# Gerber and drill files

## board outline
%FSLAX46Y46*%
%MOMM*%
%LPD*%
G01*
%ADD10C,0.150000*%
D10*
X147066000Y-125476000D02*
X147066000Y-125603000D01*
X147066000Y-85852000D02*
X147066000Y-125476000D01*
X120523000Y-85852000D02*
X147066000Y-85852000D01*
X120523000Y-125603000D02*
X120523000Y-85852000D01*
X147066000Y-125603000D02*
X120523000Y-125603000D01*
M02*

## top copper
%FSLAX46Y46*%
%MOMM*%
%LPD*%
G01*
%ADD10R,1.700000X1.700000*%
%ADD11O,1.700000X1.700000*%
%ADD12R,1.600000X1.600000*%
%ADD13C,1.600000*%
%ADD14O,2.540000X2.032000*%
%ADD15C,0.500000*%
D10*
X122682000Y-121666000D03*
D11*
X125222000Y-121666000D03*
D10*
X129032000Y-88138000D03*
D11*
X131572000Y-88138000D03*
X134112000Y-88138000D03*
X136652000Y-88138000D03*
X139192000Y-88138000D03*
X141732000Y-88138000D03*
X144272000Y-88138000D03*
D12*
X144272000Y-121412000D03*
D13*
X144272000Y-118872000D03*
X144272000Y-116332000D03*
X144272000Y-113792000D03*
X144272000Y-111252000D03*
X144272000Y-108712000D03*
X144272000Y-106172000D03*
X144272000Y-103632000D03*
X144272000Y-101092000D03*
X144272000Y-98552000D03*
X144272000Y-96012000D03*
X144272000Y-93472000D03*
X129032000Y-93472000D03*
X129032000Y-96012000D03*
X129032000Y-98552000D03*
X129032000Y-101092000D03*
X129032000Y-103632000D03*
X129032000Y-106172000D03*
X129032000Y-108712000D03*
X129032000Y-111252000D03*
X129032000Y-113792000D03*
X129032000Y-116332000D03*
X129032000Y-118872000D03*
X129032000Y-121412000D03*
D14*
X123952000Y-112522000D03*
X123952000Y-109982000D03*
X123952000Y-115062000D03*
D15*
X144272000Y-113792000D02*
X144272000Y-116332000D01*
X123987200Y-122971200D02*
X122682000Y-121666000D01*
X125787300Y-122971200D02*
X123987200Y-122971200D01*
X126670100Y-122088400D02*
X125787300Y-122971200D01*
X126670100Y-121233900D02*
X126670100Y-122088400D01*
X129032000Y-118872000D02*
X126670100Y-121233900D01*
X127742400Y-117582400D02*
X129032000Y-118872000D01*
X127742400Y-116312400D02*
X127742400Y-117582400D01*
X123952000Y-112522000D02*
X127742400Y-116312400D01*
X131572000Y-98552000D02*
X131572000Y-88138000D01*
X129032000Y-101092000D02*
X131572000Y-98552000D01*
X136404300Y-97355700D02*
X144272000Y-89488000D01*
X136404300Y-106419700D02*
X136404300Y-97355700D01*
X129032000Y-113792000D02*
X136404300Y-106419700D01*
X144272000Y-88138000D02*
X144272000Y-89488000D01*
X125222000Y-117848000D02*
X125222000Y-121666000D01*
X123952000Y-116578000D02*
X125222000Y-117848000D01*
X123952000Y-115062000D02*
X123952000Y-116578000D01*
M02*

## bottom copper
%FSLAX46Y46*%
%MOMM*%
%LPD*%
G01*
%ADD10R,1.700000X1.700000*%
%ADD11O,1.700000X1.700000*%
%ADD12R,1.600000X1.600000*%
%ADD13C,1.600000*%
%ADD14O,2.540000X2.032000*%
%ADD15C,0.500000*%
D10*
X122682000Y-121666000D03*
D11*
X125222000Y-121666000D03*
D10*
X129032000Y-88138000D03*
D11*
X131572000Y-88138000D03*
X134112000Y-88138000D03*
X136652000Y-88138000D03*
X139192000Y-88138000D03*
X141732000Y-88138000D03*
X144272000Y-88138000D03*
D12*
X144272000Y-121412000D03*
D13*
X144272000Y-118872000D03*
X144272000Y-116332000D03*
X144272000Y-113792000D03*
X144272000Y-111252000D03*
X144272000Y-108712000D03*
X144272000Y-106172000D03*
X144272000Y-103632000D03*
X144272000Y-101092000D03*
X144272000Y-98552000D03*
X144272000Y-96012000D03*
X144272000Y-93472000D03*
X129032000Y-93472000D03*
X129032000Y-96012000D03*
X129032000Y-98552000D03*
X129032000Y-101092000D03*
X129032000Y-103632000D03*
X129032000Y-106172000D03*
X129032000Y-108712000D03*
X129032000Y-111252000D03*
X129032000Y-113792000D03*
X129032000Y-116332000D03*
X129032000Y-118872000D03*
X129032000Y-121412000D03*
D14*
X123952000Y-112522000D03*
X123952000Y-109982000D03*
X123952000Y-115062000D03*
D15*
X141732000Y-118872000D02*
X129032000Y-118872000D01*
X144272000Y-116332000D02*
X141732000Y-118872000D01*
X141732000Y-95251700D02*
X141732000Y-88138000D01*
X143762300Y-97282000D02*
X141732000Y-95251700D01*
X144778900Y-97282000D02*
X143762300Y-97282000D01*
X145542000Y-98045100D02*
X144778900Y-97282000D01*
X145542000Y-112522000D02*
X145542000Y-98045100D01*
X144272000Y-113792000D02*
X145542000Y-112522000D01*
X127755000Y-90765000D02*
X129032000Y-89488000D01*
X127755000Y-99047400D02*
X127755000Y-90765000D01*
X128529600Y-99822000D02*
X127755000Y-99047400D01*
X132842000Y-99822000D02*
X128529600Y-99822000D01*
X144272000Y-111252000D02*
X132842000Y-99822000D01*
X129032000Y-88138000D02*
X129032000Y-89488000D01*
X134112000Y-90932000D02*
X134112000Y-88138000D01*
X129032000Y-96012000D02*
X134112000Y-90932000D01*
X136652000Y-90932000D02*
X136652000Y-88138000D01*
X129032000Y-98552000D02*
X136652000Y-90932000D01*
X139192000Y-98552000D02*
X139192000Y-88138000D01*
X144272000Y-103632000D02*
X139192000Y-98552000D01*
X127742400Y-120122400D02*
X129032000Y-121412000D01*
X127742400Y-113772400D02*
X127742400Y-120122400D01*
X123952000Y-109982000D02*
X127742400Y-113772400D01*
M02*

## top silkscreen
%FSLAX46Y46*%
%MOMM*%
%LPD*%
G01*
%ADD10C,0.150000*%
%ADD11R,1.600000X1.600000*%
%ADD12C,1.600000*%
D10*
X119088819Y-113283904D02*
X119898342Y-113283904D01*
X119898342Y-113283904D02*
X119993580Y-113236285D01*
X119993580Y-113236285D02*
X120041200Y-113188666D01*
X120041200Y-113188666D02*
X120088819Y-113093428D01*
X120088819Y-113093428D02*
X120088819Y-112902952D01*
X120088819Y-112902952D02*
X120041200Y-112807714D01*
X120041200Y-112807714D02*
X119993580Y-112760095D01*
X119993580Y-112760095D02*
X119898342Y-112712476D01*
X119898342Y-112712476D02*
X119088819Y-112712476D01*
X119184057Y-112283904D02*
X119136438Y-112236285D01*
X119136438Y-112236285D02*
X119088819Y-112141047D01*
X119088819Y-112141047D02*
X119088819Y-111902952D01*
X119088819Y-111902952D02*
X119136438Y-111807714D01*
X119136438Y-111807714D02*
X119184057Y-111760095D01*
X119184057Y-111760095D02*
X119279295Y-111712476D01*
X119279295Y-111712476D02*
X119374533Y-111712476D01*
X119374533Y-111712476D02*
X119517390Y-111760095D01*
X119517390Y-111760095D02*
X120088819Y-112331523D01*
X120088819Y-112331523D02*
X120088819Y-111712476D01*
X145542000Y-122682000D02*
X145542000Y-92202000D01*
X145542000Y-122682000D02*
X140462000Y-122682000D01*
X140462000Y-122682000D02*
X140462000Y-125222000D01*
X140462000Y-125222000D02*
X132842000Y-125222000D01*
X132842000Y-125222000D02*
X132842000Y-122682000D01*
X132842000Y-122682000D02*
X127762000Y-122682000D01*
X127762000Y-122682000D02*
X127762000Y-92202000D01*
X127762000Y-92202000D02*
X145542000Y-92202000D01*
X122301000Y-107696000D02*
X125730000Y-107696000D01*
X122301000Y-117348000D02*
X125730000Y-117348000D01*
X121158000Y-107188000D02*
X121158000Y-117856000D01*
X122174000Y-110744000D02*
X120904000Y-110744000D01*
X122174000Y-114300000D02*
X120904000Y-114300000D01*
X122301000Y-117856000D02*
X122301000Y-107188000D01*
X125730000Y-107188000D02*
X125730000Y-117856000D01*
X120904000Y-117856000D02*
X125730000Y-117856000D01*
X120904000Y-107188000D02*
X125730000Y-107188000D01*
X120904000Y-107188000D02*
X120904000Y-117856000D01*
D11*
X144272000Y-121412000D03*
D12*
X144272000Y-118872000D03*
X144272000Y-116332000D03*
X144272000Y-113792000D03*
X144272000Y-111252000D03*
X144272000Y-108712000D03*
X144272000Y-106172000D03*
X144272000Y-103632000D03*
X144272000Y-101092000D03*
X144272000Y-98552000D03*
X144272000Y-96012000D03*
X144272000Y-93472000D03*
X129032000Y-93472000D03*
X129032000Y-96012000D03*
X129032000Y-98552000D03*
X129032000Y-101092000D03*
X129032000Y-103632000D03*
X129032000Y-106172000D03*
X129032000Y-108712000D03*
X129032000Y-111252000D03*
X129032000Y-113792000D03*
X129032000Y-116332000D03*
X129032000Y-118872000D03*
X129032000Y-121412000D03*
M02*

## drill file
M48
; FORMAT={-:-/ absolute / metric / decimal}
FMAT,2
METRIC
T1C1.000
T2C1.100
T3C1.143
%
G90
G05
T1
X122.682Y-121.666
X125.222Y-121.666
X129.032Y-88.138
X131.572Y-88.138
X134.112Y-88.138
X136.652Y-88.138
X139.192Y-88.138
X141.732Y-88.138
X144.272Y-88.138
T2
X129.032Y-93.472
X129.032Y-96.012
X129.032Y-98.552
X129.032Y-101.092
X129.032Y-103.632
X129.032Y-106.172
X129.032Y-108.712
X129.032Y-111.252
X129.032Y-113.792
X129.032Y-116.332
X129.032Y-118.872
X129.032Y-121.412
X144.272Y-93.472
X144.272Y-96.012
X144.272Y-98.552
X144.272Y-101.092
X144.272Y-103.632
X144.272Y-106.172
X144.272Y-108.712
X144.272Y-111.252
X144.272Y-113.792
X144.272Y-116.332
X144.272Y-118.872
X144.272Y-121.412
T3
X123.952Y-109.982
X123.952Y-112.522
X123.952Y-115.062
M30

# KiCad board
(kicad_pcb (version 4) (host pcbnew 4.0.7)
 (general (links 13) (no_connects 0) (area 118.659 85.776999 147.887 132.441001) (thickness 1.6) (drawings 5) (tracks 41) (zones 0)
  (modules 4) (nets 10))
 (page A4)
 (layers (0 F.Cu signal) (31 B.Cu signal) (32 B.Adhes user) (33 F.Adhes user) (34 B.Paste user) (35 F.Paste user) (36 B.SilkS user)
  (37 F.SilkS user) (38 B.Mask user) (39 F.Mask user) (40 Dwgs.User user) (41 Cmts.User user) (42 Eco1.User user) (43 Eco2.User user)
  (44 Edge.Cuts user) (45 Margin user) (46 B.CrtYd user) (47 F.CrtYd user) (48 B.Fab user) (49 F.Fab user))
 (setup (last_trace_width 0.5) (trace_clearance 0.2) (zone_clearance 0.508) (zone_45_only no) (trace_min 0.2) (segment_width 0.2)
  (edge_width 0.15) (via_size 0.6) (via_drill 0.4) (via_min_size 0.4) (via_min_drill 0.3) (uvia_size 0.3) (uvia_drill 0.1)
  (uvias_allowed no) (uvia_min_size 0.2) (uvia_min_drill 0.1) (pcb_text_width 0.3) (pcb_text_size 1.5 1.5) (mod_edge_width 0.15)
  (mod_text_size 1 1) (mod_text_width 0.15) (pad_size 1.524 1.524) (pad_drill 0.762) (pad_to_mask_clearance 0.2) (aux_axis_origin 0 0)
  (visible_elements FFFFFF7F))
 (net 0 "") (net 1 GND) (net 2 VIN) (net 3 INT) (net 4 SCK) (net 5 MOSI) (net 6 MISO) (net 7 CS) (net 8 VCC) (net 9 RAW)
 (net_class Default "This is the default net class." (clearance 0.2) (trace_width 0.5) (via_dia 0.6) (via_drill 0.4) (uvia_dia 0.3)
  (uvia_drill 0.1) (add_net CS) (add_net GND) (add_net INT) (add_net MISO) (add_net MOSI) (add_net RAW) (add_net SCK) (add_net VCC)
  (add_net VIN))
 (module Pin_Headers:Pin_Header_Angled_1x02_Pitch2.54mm (layer B.Cu) (at 122.682 121.666 270)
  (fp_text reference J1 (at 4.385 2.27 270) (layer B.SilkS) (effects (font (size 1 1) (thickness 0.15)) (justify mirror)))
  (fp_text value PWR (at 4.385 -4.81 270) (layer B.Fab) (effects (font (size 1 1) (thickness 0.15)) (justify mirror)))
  (pad 1 thru_hole rect (at 0 0 270) (size 1.7 1.7) (drill 1) (layers *.Cu *.Mask) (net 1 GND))
  (pad 2 thru_hole oval (at 0 -2.54 270) (size 1.7 1.7) (drill 1) (layers *.Cu *.Mask) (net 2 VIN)))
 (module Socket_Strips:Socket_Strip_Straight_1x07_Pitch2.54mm (layer B.Cu) (at 129.032 88.138 270)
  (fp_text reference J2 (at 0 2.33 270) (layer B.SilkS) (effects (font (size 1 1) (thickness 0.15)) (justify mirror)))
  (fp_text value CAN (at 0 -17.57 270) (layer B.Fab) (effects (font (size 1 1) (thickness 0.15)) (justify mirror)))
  (pad 1 thru_hole rect (at 0 0 270) (size 1.7 1.7) (drill 1) (layers *.Cu *.Mask) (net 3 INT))
  (pad 2 thru_hole oval (at 0 -2.54 270) (size 1.7 1.7) (drill 1) (layers *.Cu *.Mask) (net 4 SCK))
  (pad 3 thru_hole oval (at 0 -5.08 270) (size 1.7 1.7) (drill 1) (layers *.Cu *.Mask) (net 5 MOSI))
  (pad 4 thru_hole oval (at 0 -7.62 270) (size 1.7 1.7) (drill 1) (layers *.Cu *.Mask) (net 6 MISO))
  (pad 5 thru_hole oval (at 0 -10.16 270) (size 1.7 1.7) (drill 1) (layers *.Cu *.Mask) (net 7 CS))
  (pad 6 thru_hole oval (at 0 -12.7 270) (size 1.7 1.7) (drill 1) (layers *.Cu *.Mask) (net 1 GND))
  (pad 7 thru_hole oval (at 0 -15.24 270) (size 1.7 1.7) (drill 1) (layers *.Cu *.Mask) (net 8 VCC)))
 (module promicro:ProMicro (layer F.Cu) (at 136.652 107.442 90)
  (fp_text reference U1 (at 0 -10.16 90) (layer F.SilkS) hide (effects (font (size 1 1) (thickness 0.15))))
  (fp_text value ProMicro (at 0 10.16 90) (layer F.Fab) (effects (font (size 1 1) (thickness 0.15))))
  (fp_line (start -15.24 8.89) (end 15.24 8.89) (layer F.SilkS) (width 0.15))
  (fp_line (start -15.24 8.89) (end -15.24 3.81) (layer F.SilkS) (width 0.15))
  (fp_line (start -15.24 3.81) (end -17.78 3.81) (layer F.SilkS) (width 0.15))
  (fp_line (start -17.78 3.81) (end -17.78 -3.81) (layer F.SilkS) (width 0.15))
  (fp_line (start -17.78 -3.81) (end -15.24 -3.81) (layer F.SilkS) (width 0.15))
  (fp_line (start -15.24 -3.81) (end -15.24 -8.89) (layer F.SilkS) (width 0.15))
  (fp_line (start -15.24 -8.89) (end 15.24 -8.89) (layer F.SilkS) (width 0.15))
  (fp_line (start 15.24 -8.89) (end 15.24 8.89) (layer F.SilkS) (width 0.15))
  (pad 1 thru_hole rect (at -13.97 7.62 90) (size 1.6 1.6) (drill 1.1) (layers *.Cu *.Mask F.SilkS))
  (pad 2 thru_hole circle (at -11.43 7.62 90) (size 1.6 1.6) (drill 1.1) (layers *.Cu *.Mask F.SilkS))
  (pad 3 thru_hole circle (at -8.89 7.62 90) (size 1.6 1.6) (drill 1.1) (layers *.Cu *.Mask F.SilkS) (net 1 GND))
  (pad 4 thru_hole circle (at -6.35 7.62 90) (size 1.6 1.6) (drill 1.1) (layers *.Cu *.Mask F.SilkS) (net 1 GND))
  (pad 5 thru_hole circle (at -3.81 7.62 90) (size 1.6 1.6) (drill 1.1) (layers *.Cu *.Mask F.SilkS) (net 3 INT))
  (pad 6 thru_hole circle (at -1.27 7.62 90) (size 1.6 1.6) (drill 1.1) (layers *.Cu *.Mask F.SilkS))
  (pad 7 thru_hole circle (at 1.27 7.62 90) (size 1.6 1.6) (drill 1.1) (layers *.Cu *.Mask F.SilkS))
  (pad 8 thru_hole circle (at 3.81 7.62 90) (size 1.6 1.6) (drill 1.1) (layers *.Cu *.Mask F.SilkS) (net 7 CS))
  (pad 9 thru_hole circle (at 6.35 7.62 90) (size 1.6 1.6) (drill 1.1) (layers *.Cu *.Mask F.SilkS))
  (pad 10 thru_hole circle (at 8.89 7.62 90) (size 1.6 1.6) (drill 1.1) (layers *.Cu *.Mask F.SilkS))
  (pad 11 thru_hole circle (at 11.43 7.62 90) (size 1.6 1.6) (drill 1.1) (layers *.Cu *.Mask F.SilkS))
  (pad 12 thru_hole circle (at 13.97 7.62 90) (size 1.6 1.6) (drill 1.1) (layers *.Cu *.Mask F.SilkS))
  (pad 13 thru_hole circle (at 13.97 -7.62 90) (size 1.6 1.6) (drill 1.1) (layers *.Cu *.Mask F.SilkS))
  (pad 14 thru_hole circle (at 11.43 -7.62 90) (size 1.6 1.6) (drill 1.1) (layers *.Cu *.Mask F.SilkS) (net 5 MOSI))
  (pad 15 thru_hole circle (at 8.89 -7.62 90) (size 1.6 1.6) (drill 1.1) (layers *.Cu *.Mask F.SilkS) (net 6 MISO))
  (pad 16 thru_hole circle (at 6.35 -7.62 90) (size 1.6 1.6) (drill 1.1) (layers *.Cu *.Mask F.SilkS) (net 4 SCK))
  (pad 17 thru_hole circle (at 3.81 -7.62 90) (size 1.6 1.6) (drill 1.1) (layers *.Cu *.Mask F.SilkS))
  (pad 18 thru_hole circle (at 1.27 -7.62 90) (size 1.6 1.6) (drill 1.1) (layers *.Cu *.Mask F.SilkS))
  (pad 19 thru_hole circle (at -1.27 -7.62 90) (size 1.6 1.6) (drill 1.1) (layers *.Cu *.Mask F.SilkS))
  (pad 20 thru_hole circle (at -3.81 -7.62 90) (size 1.6 1.6) (drill 1.1) (layers *.Cu *.Mask F.SilkS))
  (pad 21 thru_hole circle (at -6.35 -7.62 90) (size 1.6 1.6) (drill 1.1) (layers *.Cu *.Mask F.SilkS) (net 8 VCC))
  (pad 22 thru_hole circle (at -8.89 -7.62 90) (size 1.6 1.6) (drill 1.1) (layers *.Cu *.Mask F.SilkS))
  (pad 23 thru_hole circle (at -11.43 -7.62 90) (size 1.6 1.6) (drill 1.1) (layers *.Cu *.Mask F.SilkS) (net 1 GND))
  (pad 24 thru_hole circle (at -13.97 -7.62 90) (size 1.6 1.6) (drill 1.1) (layers *.Cu *.Mask F.SilkS) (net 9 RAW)))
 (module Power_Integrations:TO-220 (layer F.Cu) (at 123.952 112.522 90)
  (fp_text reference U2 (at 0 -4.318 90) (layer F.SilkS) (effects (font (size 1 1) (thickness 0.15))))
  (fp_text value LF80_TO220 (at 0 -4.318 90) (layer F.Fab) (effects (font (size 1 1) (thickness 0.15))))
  (fp_line (start 4.826 -1.651) (end 4.826 1.778) (layer F.SilkS) (width 0.15))
  (fp_line (start -4.826 -1.651) (end -4.826 1.778) (layer F.SilkS) (width 0.15))
  (fp_line (start 5.334 -2.794) (end -5.334 -2.794) (layer F.SilkS) (width 0.15))
  (fp_line (start 1.778 -1.778) (end 1.778 -3.048) (layer F.SilkS) (width 0.15))
  (fp_line (start -1.778 -1.778) (end -1.778 -3.048) (layer F.SilkS) (width 0.15))
  (fp_line (start -5.334 -1.651) (end 5.334 -1.651) (layer F.SilkS) (width 0.15))
  (fp_line (start 5.334 1.778) (end -5.334 1.778) (layer F.SilkS) (width 0.15))
  (fp_line (start -5.334 -3.048) (end -5.334 1.778) (layer F.SilkS) (width 0.15))
  (fp_line (start 5.334 -3.048) (end 5.334 1.778) (layer F.SilkS) (width 0.15))
  (fp_line (start 5.334 -3.048) (end -5.334 -3.048) (layer F.SilkS) (width 0.15))
  (pad 2 thru_hole oval (at 0 0 90) (size 2.032 2.54) (drill 1.143) (layers *.Cu *.Mask) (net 1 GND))
  (pad 3 thru_hole oval (at 2.54 0 90) (size 2.032 2.54) (drill 1.143) (layers *.Cu *.Mask) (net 9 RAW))
  (pad 1 thru_hole oval (at -2.54 0 90) (size 2.032 2.54) (drill 1.143) (layers *.Cu *.Mask) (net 2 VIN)))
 (gr_line (start 147.066 125.476) (end 147.066 125.603) (angle 90) (layer Edge.Cuts) (width 0.15))
 (gr_line (start 147.066 85.852) (end 147.066 125.476) (angle 90) (layer Edge.Cuts) (width 0.15))
 (gr_line (start 120.523 85.852) (end 147.066 85.852) (angle 90) (layer Edge.Cuts) (width 0.15))
 (gr_line (start 120.523 125.603) (end 120.523 85.852) (angle 90) (layer Edge.Cuts) (width 0.15))
 (gr_line (start 147.066 125.603) (end 120.523 125.603) (angle 90) (layer Edge.Cuts) (width 0.15))
 (segment (start 141.732 118.872) (end 129.032 118.872) (width 0.5) (layer B.Cu) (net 1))
 (segment (start 144.272 116.332) (end 141.732 118.872) (width 0.5) (layer B.Cu) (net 1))
 (segment (start 144.272 113.792) (end 144.272 116.332) (width 0.5) (layer F.Cu) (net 1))
 (segment (start 123.9872 122.9712) (end 122.682 121.666) (width 0.5) (layer F.Cu) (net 1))
 (segment (start 125.7873 122.9712) (end 123.9872 122.9712) (width 0.5) (layer F.Cu) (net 1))
 (segment (start 126.6701 122.0884) (end 125.7873 122.9712) (width 0.5) (layer F.Cu) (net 1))
 (segment (start 126.6701 121.2339) (end 126.6701 122.0884) (width 0.5) (layer F.Cu) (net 1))
 (segment (start 129.032 118.872) (end 126.6701 121.2339) (width 0.5) (layer F.Cu) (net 1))
 (segment (start 127.7424 117.5824) (end 129.032 118.872) (width 0.5) (layer F.Cu) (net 1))
 (segment (start 127.7424 116.3124) (end 127.7424 117.5824) (width 0.5) (layer F.Cu) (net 1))
 (segment (start 123.952 112.522) (end 127.7424 116.3124) (width 0.5) (layer F.Cu) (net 1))
 (segment (start 141.732 95.2517) (end 141.732 88.138) (width 0.5) (layer B.Cu) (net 1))
 (segment (start 143.7623 97.282) (end 141.732 95.2517) (width 0.5) (layer B.Cu) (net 1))
 (segment (start 144.7789 97.282) (end 143.7623 97.282) (width 0.5) (layer B.Cu) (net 1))
 (segment (start 145.542 98.0451) (end 144.7789 97.282) (width 0.5) (layer B.Cu) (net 1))
 (segment (start 145.542 112.522) (end 145.542 98.0451) (width 0.5) (layer B.Cu) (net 1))
 (segment (start 144.272 113.792) (end 145.542 112.522) (width 0.5) (layer B.Cu) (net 1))
 (segment (start 127.755 90.765) (end 129.032 89.488) (width 0.5) (layer B.Cu) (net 3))
 (segment (start 127.755 99.0474) (end 127.755 90.765) (width 0.5) (layer B.Cu) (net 3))
 (segment (start 128.5296 99.822) (end 127.755 99.0474) (width 0.5) (layer B.Cu) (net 3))
 (segment (start 132.842 99.822) (end 128.5296 99.822) (width 0.5) (layer B.Cu) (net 3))
 (segment (start 144.272 111.252) (end 132.842 99.822) (width 0.5) (layer B.Cu) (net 3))
 (segment (start 129.032 88.138) (end 129.032 89.488) (width 0.5) (layer B.Cu) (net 3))
 (segment (start 131.572 98.552) (end 131.572 88.138) (width 0.5) (layer F.Cu) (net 4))
 (segment (start 129.032 101.092) (end 131.572 98.552) (width 0.5) (layer F.Cu) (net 4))
 (segment (start 134.112 90.932) (end 134.112 88.138) (width 0.5) (layer B.Cu) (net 5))
 (segment (start 129.032 96.012) (end 134.112 90.932) (width 0.5) (layer B.Cu) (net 5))
 (segment (start 136.652 90.932) (end 136.652 88.138) (width 0.5) (layer B.Cu) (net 6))
 (segment (start 129.032 98.552) (end 136.652 90.932) (width 0.5) (layer B.Cu) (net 6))
 (segment (start 139.192 98.552) (end 139.192 88.138) (width 0.5) (layer B.Cu) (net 7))
 (segment (start 144.272 103.632) (end 139.192 98.552) (width 0.5) (layer B.Cu) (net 7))
 (segment (start 136.4043 97.3557) (end 144.272 89.488) (width 0.5) (layer F.Cu) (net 8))
 (segment (start 136.4043 106.4197) (end 136.4043 97.3557) (width 0.5) (layer F.Cu) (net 8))
 (segment (start 129.032 113.792) (end 136.4043 106.4197) (width 0.5) (layer F.Cu) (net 8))
 (segment (start 144.272 88.138) (end 144.272 89.488) (width 0.5) (layer F.Cu) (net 8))
 (segment (start 125.222 117.848) (end 125.222 121.666) (width 0.5) (layer F.Cu) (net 2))
 (segment (start 123.952 116.578) (end 125.222 117.848) (width 0.5) (layer F.Cu) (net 2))
 (segment (start 123.952 115.062) (end 123.952 116.578) (width 0.5) (layer F.Cu) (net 2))
 (segment (start 127.7424 120.1224) (end 129.032 121.412) (width 0.5) (layer B.Cu) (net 9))
 (segment (start 127.7424 113.7724) (end 127.7424 120.1224) (width 0.5) (layer B.Cu) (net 9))
 (segment (start 123.952 109.982) (end 127.7424 113.7724) (width 0.5) (layer B.Cu) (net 9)))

